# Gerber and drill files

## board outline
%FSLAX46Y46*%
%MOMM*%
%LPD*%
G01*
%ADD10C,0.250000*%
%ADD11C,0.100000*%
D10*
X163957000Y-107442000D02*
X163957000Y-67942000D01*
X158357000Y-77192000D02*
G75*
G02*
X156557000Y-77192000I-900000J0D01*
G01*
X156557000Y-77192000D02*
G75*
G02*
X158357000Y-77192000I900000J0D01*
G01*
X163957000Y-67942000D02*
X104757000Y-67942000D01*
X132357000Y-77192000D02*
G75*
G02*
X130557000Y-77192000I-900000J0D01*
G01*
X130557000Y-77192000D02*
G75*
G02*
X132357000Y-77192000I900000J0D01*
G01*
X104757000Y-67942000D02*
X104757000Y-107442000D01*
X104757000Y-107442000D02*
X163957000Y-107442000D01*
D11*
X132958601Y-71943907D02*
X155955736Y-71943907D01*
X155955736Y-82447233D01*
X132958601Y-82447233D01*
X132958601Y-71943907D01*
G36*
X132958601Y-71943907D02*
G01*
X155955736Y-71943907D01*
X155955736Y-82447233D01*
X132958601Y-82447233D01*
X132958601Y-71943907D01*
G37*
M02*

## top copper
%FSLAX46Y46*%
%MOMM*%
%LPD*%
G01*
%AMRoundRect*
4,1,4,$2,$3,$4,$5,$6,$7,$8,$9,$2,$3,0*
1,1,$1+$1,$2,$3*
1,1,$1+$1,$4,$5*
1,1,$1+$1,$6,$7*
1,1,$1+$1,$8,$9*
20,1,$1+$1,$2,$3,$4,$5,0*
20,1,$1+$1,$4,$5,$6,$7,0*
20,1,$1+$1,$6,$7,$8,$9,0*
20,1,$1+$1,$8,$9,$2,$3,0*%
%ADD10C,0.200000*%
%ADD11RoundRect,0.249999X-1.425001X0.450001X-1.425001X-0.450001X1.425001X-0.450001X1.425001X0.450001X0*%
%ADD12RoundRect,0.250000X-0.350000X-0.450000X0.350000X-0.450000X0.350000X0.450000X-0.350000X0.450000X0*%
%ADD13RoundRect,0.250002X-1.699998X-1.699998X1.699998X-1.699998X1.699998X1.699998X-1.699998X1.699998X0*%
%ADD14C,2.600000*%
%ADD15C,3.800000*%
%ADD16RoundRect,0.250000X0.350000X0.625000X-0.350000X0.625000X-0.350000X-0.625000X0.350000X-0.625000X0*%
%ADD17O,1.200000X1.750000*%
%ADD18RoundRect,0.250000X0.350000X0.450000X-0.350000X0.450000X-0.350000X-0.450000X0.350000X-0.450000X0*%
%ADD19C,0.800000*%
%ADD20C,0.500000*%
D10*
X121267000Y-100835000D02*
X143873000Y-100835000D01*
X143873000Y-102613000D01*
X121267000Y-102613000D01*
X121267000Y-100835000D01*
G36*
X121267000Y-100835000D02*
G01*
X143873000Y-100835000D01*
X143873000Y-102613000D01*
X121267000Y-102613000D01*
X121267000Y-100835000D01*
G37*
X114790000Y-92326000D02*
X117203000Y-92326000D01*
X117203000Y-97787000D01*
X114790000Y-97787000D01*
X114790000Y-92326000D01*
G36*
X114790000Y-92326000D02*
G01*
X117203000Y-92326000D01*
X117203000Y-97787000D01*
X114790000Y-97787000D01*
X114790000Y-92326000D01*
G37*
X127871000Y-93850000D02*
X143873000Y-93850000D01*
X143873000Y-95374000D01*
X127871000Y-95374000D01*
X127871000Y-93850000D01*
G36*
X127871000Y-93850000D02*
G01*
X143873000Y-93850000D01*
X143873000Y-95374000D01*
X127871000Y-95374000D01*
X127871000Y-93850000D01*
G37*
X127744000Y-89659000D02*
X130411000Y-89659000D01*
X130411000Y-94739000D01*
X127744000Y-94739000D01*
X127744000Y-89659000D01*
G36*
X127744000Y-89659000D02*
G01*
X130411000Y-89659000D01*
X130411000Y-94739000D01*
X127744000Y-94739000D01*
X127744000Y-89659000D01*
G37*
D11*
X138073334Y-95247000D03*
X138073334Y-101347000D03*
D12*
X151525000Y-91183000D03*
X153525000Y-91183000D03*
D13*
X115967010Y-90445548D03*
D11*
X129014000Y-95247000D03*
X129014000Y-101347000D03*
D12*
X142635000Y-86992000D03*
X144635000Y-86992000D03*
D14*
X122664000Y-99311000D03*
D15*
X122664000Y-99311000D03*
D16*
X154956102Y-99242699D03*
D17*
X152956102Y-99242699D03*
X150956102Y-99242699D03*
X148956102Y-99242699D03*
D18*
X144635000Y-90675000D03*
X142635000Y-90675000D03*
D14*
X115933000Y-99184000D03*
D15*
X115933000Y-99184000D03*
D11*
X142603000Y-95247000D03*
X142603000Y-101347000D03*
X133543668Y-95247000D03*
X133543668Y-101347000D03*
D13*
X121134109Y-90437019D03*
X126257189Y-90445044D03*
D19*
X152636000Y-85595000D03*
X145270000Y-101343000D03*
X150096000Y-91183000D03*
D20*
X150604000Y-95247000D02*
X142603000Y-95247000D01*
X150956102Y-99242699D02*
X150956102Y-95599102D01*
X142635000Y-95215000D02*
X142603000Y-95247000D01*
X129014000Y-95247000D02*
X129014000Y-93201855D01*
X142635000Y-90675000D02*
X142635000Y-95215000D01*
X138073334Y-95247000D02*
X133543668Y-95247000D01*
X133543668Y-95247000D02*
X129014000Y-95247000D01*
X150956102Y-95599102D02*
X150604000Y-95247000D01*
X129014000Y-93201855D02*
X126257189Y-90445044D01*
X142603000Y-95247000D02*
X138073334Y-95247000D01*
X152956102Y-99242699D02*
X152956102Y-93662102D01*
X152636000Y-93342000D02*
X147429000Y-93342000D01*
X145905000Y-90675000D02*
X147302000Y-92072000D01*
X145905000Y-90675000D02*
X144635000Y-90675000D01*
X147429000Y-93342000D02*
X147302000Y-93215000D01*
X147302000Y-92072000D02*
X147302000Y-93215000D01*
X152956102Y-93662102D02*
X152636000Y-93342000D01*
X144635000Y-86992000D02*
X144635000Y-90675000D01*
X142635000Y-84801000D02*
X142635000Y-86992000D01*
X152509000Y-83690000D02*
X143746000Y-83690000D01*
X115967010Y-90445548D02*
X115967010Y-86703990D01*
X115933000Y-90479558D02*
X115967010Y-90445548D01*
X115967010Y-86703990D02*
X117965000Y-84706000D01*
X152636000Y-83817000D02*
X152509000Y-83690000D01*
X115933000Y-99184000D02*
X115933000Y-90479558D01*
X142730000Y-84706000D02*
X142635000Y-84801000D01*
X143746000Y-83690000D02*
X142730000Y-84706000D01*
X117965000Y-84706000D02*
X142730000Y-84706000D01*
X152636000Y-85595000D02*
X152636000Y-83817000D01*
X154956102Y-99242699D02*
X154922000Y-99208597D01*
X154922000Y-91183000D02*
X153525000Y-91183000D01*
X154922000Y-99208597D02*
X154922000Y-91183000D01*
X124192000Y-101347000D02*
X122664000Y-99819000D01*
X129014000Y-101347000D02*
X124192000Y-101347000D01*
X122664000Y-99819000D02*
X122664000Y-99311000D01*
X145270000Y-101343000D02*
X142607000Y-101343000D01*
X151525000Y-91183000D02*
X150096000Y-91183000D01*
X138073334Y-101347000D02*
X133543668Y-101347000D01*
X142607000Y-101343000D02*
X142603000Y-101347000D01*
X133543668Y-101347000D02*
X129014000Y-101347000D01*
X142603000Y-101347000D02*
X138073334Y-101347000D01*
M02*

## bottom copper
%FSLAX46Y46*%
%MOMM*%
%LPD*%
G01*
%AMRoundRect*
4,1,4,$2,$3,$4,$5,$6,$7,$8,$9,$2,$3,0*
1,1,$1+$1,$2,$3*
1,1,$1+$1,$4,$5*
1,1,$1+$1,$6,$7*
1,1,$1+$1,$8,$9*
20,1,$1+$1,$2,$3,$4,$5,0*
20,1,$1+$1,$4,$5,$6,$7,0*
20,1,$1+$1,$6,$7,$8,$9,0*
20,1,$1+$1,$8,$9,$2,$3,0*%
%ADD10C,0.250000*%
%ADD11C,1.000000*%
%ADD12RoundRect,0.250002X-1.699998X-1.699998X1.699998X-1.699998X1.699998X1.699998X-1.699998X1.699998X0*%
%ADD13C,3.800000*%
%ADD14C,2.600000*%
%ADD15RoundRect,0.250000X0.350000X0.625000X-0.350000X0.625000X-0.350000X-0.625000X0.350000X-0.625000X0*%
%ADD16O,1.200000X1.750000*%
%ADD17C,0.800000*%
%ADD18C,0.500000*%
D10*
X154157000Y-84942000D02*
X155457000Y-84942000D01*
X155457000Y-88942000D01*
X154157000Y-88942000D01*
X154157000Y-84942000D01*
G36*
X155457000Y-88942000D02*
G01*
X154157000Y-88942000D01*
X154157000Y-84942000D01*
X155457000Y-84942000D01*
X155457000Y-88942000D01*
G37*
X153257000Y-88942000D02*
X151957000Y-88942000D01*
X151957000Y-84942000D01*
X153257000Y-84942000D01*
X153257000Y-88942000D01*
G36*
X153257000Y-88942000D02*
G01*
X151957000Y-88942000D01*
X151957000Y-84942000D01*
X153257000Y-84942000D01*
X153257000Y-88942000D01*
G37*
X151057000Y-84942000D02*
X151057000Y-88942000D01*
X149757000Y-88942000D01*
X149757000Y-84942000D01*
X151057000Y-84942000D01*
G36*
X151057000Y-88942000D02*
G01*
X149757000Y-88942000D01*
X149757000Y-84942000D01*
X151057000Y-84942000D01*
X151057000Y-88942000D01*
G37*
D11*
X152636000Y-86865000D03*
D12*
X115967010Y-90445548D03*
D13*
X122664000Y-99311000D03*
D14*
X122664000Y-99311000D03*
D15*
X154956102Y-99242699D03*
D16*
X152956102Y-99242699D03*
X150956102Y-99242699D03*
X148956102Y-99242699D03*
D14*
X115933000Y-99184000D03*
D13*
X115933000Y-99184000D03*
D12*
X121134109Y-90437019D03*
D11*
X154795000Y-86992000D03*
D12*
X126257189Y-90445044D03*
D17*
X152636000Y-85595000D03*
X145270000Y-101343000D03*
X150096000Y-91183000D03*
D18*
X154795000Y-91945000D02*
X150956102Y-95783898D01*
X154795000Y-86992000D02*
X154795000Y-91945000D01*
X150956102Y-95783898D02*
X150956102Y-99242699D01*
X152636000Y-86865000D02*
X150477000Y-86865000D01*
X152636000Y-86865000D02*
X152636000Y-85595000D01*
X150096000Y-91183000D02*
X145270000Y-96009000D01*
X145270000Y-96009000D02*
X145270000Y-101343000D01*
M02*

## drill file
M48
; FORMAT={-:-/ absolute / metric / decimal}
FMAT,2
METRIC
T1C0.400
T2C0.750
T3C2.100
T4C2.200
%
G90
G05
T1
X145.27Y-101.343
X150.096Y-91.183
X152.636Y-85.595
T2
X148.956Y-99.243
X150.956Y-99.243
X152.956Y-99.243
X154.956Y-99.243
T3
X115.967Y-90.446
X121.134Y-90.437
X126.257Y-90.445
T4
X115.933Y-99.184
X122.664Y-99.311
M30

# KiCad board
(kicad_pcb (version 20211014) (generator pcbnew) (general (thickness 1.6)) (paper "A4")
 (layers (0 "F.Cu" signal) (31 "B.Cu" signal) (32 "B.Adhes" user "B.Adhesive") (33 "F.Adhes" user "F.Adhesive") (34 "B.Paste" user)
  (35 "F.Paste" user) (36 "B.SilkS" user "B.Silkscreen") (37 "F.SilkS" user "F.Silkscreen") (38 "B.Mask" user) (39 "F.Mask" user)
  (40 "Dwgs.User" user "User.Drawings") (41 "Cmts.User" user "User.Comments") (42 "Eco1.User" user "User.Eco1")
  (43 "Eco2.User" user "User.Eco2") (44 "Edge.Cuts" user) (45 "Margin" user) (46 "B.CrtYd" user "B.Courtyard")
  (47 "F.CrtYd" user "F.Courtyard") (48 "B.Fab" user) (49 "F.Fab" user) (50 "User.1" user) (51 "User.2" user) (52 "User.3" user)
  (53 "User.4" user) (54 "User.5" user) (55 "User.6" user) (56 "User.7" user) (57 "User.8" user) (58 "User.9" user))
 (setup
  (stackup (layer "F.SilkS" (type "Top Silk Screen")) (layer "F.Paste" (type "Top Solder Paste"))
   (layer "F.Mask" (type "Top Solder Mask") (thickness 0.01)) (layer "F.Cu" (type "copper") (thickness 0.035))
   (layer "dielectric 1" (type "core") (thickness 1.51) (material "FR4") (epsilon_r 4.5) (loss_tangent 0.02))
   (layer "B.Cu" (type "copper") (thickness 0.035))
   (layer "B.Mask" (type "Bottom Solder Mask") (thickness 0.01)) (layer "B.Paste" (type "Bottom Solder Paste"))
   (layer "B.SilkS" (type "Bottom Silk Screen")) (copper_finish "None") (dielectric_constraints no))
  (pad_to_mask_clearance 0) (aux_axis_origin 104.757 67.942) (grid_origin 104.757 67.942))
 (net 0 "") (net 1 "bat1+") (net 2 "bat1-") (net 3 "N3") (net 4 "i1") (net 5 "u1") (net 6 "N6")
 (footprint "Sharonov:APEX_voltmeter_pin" (layer "F.Cu") (at 152.636 86.865)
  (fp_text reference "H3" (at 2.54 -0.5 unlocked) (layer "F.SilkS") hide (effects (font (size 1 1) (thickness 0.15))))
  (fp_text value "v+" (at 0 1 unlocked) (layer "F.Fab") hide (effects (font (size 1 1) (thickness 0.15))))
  (pad "1" smd circle (at 0 0) (size 1 1) (layers "B.Cu") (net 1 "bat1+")))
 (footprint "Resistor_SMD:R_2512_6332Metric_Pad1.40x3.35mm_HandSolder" (layer "F.Cu") (at 138.073334 98.297 -90)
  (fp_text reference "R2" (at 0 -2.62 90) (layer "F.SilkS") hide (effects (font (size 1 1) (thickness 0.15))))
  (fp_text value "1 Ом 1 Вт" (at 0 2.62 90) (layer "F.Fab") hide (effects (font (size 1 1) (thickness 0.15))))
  (pad "1" smd roundrect locked (at -3.05 0 270) (size 1.4 3.35) (layers "F.Cu" "F.Paste" "F.Mask") (roundrect_rratio 0.1785707143)
   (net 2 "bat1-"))
  (pad "2" smd roundrect locked (at 3.05 0 270) (size 1.4 3.35) (layers "F.Cu" "F.Paste" "F.Mask") (roundrect_rratio 0.1785707143)
   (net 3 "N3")))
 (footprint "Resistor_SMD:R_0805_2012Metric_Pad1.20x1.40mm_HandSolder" (layer "F.Cu") (at 152.525 91.183)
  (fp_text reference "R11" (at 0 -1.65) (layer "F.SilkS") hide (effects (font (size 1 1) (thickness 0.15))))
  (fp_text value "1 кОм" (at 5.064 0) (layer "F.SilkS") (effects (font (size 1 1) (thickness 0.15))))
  (pad "1" smd roundrect locked (at -1 0) (size 1.2 1.4) (layers "F.Cu" "F.Paste" "F.Mask") (roundrect_rratio 0.2083333333) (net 3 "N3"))
  (pad "2" smd roundrect locked (at 1 0) (size 1.2 1.4) (layers "F.Cu" "F.Paste" "F.Mask") (roundrect_rratio 0.2083333333) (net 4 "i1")))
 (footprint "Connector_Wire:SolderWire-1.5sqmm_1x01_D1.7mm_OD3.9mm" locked (layer "F.Cu") (at 115.96701 90.445548)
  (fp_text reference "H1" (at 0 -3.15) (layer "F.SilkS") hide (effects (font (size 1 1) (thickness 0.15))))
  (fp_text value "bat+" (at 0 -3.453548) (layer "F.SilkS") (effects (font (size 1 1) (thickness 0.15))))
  (pad "1" thru_hole roundrect locked (at 0 0) (size 3.9 3.9) (drill 2.1) (layers *.Cu *.Mask) (roundrect_rratio 0.06410307692)
   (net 1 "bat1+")))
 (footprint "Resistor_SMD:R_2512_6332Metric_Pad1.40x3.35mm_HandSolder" (layer "F.Cu") (at 129.014 98.297 -90)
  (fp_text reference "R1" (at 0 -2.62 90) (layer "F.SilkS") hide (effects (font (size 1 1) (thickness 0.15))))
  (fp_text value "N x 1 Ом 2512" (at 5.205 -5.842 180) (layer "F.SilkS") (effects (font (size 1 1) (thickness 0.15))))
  (pad "1" smd roundrect locked (at -3.05 0 270) (size 1.4 3.35) (layers "F.Cu" "F.Paste" "F.Mask") (roundrect_rratio 0.1785707143)
   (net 2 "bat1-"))
  (pad "2" smd roundrect locked (at 3.05 0 270) (size 1.4 3.35) (layers "F.Cu" "F.Paste" "F.Mask") (roundrect_rratio 0.1785707143)
   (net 3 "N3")))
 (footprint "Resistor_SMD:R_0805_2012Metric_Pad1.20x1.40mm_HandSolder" (layer "F.Cu") (at 143.635 86.992)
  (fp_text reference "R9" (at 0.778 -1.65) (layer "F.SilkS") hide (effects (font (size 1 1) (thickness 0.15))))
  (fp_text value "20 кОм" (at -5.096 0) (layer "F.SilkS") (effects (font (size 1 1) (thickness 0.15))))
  (pad "1" smd roundrect locked (at -1 0) (size 1.2 1.4) (layers "F.Cu" "F.Paste" "F.Mask") (roundrect_rratio 0.2083333333) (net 1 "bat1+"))
  (pad "2" smd roundrect locked (at 1 0) (size 1.2 1.4) (layers "F.Cu" "F.Paste" "F.Mask") (roundrect_rratio 0.2083333333) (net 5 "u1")))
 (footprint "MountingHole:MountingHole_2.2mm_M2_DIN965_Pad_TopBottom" (layer "F.Cu") (at 122.664 99.311)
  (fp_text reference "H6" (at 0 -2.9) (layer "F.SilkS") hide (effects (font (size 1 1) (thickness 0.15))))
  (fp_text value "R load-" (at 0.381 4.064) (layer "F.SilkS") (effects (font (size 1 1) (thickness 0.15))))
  (pad "1" connect circle locked (at 0 0) (size 3.8 3.8) (layers "B.Cu" "B.Mask") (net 3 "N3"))
  (pad "1" thru_hole circle locked (at 0 0) (size 2.6 2.6) (drill 2.2) (layers *.Cu *.Mask) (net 3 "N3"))
  (pad "1" connect circle locked (at 0 0) (size 3.8 3.8) (layers "F.Cu" "F.Mask") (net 3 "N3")))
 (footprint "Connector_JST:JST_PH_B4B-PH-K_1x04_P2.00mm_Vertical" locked (layer "F.Cu") (at 154.956102 99.242699 180)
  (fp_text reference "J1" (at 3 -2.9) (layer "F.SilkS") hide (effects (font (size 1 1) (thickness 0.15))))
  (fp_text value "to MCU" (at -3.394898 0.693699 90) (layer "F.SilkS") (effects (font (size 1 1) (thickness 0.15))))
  (pad "1" thru_hole roundrect locked (at 0 0 180) (size 1.2 1.75) (drill 0.75) (layers *.Cu *.Mask) (roundrect_rratio 0.2083333333)
   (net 4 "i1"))
  (pad "2" thru_hole oval locked (at 2 0 180) (size 1.2 1.75) (drill 0.75) (layers *.Cu *.Mask) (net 5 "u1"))
  (pad "3" thru_hole oval locked (at 4 0 180) (size 1.2 1.75) (drill 0.75) (layers *.Cu *.Mask) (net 2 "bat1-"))
  (pad "4" thru_hole oval locked (at 6 0 180) (size 1.2 1.75) (drill 0.75) (layers *.Cu *.Mask) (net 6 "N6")))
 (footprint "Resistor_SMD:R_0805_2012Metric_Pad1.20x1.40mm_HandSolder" (layer "F.Cu") (at 143.635 90.675 180)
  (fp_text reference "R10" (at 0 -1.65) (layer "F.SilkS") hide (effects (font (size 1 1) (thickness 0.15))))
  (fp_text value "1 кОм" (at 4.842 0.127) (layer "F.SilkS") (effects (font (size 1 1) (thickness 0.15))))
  (pad "1" smd roundrect locked (at -1 0 180) (size 1.2 1.4) (layers "F.Cu" "F.Paste" "F.Mask") (roundrect_rratio 0.2083333333) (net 5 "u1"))
  (pad "2" smd roundrect locked (at 1 0 180) (size 1.2 1.4) (layers "F.Cu" "F.Paste" "F.Mask") (roundrect_rratio 0.2083333333)
   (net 2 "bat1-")))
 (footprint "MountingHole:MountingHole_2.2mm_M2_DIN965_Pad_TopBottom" (layer "F.Cu") (at 115.933 99.184)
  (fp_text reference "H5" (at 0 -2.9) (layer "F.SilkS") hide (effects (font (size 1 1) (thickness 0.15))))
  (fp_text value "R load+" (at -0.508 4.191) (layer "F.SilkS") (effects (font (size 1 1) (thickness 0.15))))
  (pad "1" thru_hole circle locked (at 0 0) (size 2.6 2.6) (drill 2.2) (layers *.Cu *.Mask) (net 1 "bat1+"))
  (pad "1" connect circle locked (at 0 0) (size 3.8 3.8) (layers "F.Cu" "F.Mask") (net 1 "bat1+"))
  (pad "1" connect circle locked (at 0 0) (size 3.8 3.8) (layers "B.Cu" "B.Mask") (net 1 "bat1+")))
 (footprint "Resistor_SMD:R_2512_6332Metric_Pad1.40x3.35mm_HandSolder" (layer "F.Cu") (at 142.603 98.297 -90)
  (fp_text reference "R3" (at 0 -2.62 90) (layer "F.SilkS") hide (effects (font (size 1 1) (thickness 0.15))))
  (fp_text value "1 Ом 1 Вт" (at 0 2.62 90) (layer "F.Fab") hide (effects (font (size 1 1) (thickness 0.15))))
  (pad "1" smd roundrect locked (at -3.05 0 270) (size 1.4 3.35) (layers "F.Cu" "F.Paste" "F.Mask") (roundrect_rratio 0.1785707143)
   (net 2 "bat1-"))
  (pad "2" smd roundrect locked (at 3.05 0 270) (size 1.4 3.35) (layers "F.Cu" "F.Paste" "F.Mask") (roundrect_rratio 0.1785707143)
   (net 3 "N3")))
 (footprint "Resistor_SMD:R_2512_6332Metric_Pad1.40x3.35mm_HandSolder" (layer "F.Cu") (at 133.543668 98.297 -90)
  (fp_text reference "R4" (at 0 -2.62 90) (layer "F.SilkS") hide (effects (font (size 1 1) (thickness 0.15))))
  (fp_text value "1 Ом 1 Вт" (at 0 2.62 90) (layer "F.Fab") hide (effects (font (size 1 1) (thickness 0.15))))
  (pad "1" smd roundrect locked (at -3.05 0 270) (size 1.4 3.35) (layers "F.Cu" "F.Paste" "F.Mask") (roundrect_rratio 0.1785707143)
   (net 2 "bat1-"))
  (pad "2" smd roundrect locked (at 3.05 0 270) (size 1.4 3.35) (layers "F.Cu" "F.Paste" "F.Mask") (roundrect_rratio 0.1785707143)
   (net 3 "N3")))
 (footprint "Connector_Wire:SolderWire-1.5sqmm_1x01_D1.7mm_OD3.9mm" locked (layer "F.Cu") (at 121.134109 90.437019)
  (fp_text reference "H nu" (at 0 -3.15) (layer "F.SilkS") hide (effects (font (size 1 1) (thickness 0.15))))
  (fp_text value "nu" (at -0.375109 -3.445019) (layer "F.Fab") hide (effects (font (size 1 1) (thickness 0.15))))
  (pad "1" thru_hole roundrect locked (at 0 0) (size 3.9 3.9) (drill 2.1) (layers *.Cu *.Mask) (roundrect_rratio 0.06410307692)))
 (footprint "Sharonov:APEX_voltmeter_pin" (layer "F.Cu") (at 154.795 86.992)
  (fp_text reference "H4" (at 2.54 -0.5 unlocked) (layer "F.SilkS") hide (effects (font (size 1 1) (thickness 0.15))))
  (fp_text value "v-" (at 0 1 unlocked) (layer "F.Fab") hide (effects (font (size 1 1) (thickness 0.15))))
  (pad "1" smd circle (at 0 0) (size 1 1) (layers "B.Cu") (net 2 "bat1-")))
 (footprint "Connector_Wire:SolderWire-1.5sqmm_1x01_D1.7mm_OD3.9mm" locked (layer "F.Cu") (at 126.257189 90.445044)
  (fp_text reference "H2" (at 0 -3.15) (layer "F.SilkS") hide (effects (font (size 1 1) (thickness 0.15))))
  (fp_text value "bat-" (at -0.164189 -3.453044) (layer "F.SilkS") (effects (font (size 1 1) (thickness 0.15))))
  (pad "1" thru_hole roundrect locked (at 0 0) (size 3.9 3.9) (drill 2.1) (layers *.Cu *.Mask) (roundrect_rratio 0.06410307692)
   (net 2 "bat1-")))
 (gr_rect (start 143.873 102.613) (end 121.267 100.835) (layer "F.Cu") (width 0.2) (fill solid))
 (gr_rect (start 114.79 92.326) (end 117.203 97.787) (layer "F.Cu") (width 0.2) (fill solid))
 (gr_rect (start 127.871 95.374) (end 143.873 93.85) (layer "F.Cu") (width 0.2) (fill solid))
 (gr_rect (start 130.411 94.739) (end 127.744 89.659) (layer "F.Cu") (width 0.2) (fill solid))
 (gr_poly locked
  (pts (xy 154.157 84.942) (xy 155.457 84.942) (xy 155.457 88.942) (xy 154.157 88.942)) (layer "B.Cu") (width 0.25) (fill solid))
 (gr_poly locked
  (pts (xy 153.257 88.942) (xy 151.957 88.942) (xy 151.957 84.942) (xy 153.257 84.942)) (layer "B.Cu") (width 0.25) (fill solid))
 (gr_poly locked
  (pts (xy 151.057 84.942) (xy 151.057 88.942) (xy 149.757 88.942) (xy 149.757 84.942)) (layer "B.Cu") (width 0.25) (fill solid))
 (gr_line locked (start 163.957 107.442) (end 163.957 67.942) (layer "Edge.Cuts") (width 0.25))
 (gr_circle locked (center 157.457 77.192) (end 158.357 77.192) (layer "Edge.Cuts") (width 0.25) (fill none))
 (gr_line locked (start 163.957 67.942) (end 104.757 67.942) (layer "Edge.Cuts") (width 0.25))
 (gr_circle locked (center 131.457 77.192) (end 132.357 77.192) (layer "Edge.Cuts") (width 0.25) (fill none))
 (gr_line locked (start 104.757 67.942) (end 104.757 107.442) (layer "Edge.Cuts") (width 0.25))
 (gr_line locked (start 104.757 107.442) (end 163.957 107.442) (layer "Edge.Cuts") (width 0.25))
 (gr_rect locked (start 132.958601 71.943907) (end 155.955736 82.447233) (layer "Edge.Cuts") (width 0.1) (fill solid))
 (segment (start 150.604 95.247) (end 142.603 95.247) (width 0.5) (layer "F.Cu") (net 2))
 (segment (start 150.956102 99.242699) (end 150.956102 95.599102) (width 0.5) (layer "F.Cu") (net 2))
 (segment (start 142.635 95.215) (end 142.603 95.247) (width 0.5) (layer "F.Cu") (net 2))
 (segment (start 129.014 95.247) (end 129.014 93.201855) (width 0.5) (layer "F.Cu") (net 2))
 (segment (start 142.635 90.675) (end 142.635 95.215) (width 0.5) (layer "F.Cu") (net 2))
 (segment (start 138.073334 95.247) (end 133.543668 95.247) (width 0.5) (layer "F.Cu") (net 2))
 (segment (start 133.543668 95.247) (end 129.014 95.247) (width 0.5) (layer "F.Cu") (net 2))
 (segment (start 150.956102 95.599102) (end 150.604 95.247) (width 0.5) (layer "F.Cu") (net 2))
 (segment (start 129.014 93.201855) (end 126.257189 90.445044) (width 0.5) (layer "F.Cu") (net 2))
 (segment (start 142.603 95.247) (end 138.073334 95.247) (width 0.5) (layer "F.Cu") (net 2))
 (segment (start 154.795 91.945) (end 150.956102 95.783898) (width 0.5) (layer "B.Cu") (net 2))
 (segment (start 154.795 86.992) (end 154.795 91.945) (width 0.5) (layer "B.Cu") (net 2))
 (segment (start 150.956102 95.783898) (end 150.956102 99.242699) (width 0.5) (layer "B.Cu") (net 2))
 (segment (start 152.956102 99.242699) (end 152.956102 93.662102) (width 0.5) (layer "F.Cu") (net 5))
 (segment (start 152.636 93.342) (end 147.429 93.342) (width 0.5) (layer "F.Cu") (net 5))
 (segment (start 145.905 90.675) (end 147.302 92.072) (width 0.5) (layer "F.Cu") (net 5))
 (segment (start 145.905 90.675) (end 144.635 90.675) (width 0.5) (layer "F.Cu") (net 5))
 (segment (start 147.429 93.342) (end 147.302 93.215) (width 0.5) (layer "F.Cu") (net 5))
 (segment (start 147.302 92.072) (end 147.302 93.215) (width 0.5) (layer "F.Cu") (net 5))
 (segment (start 152.956102 93.662102) (end 152.636 93.342) (width 0.5) (layer "F.Cu") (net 5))
 (segment (start 144.635 86.992) (end 144.635 90.675) (width 0.5) (layer "F.Cu") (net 5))
 (segment (start 142.635 84.801) (end 142.635 86.992) (width 0.5) (layer "F.Cu") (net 1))
 (segment (start 152.509 83.69) (end 143.746 83.69) (width 0.5) (layer "F.Cu") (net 1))
 (segment (start 115.96701 90.445548) (end 115.96701 86.70399) (width 0.5) (layer "F.Cu") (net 1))
 (segment (start 115.933 90.479558) (end 115.96701 90.445548) (width 0.5) (layer "F.Cu") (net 1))
 (segment (start 115.96701 86.70399) (end 117.965 84.706) (width 0.5) (layer "F.Cu") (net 1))
 (segment (start 152.636 83.817) (end 152.509 83.69) (width 0.5) (layer "F.Cu") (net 1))
 (segment (start 115.933 99.184) (end 115.933 90.479558) (width 0.5) (layer "F.Cu") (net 1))
 (segment (start 142.73 84.706) (end 142.635 84.801) (width 0.5) (layer "F.Cu") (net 1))
 (segment (start 143.746 83.69) (end 142.73 84.706) (width 0.5) (layer "F.Cu") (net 1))
 (segment (start 117.965 84.706) (end 142.73 84.706) (width 0.5) (layer "F.Cu") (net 1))
 (segment (start 152.636 85.595) (end 152.636 83.817) (width 0.5) (layer "F.Cu") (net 1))
 (via (at 152.636 85.595) (size 0.8) (drill 0.4) (layers "F.Cu" "B.Cu") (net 1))
 (segment (start 152.636 86.865) (end 150.477 86.865) (width 0.5) (layer "B.Cu") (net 1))
 (segment (start 152.636 86.865) (end 152.636 85.595) (width 0.5) (layer "B.Cu") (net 1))
 (segment (start 154.956102 99.242699) (end 154.922 99.208597) (width 0.5) (layer "F.Cu") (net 4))
 (segment (start 154.922 91.183) (end 153.525 91.183) (width 0.5) (layer "F.Cu") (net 4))
 (segment (start 154.922 99.208597) (end 154.922 91.183) (width 0.5) (layer "F.Cu") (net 4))
 (segment (start 124.192 101.347) (end 122.664 99.819) (width 0.5) (layer "F.Cu") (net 3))
 (segment (start 129.014 101.347) (end 124.192 101.347) (width 0.5) (layer "F.Cu") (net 3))
 (segment (start 122.664 99.819) (end 122.664 99.311) (width 0.5) (layer "F.Cu") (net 3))
 (segment (start 145.27 101.343) (end 142.607 101.343) (width 0.5) (layer "F.Cu") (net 3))
 (segment (start 151.525 91.183) (end 150.096 91.183) (width 0.5) (layer "F.Cu") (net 3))
 (segment (start 138.073334 101.347) (end 133.543668 101.347) (width 0.5) (layer "F.Cu") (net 3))
 (segment (start 142.607 101.343) (end 142.603 101.347) (width 0.5) (layer "F.Cu") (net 3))
 (segment (start 133.543668 101.347) (end 129.014 101.347) (width 0.5) (layer "F.Cu") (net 3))
 (segment (start 142.603 101.347) (end 138.073334 101.347) (width 0.5) (layer "F.Cu") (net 3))
 (via (at 145.27 101.343) (size 0.8) (drill 0.4) (layers "F.Cu" "B.Cu") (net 3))
 (via (at 150.096 91.183) (size 0.8) (drill 0.4) (layers "F.Cu" "B.Cu") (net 3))
 (segment (start 150.096 91.183) (end 145.27 96.009) (width 0.5) (layer "B.Cu") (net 3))
 (segment (start 145.27 96.009) (end 145.27 101.343) (width 0.5) (layer "B.Cu") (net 3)))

